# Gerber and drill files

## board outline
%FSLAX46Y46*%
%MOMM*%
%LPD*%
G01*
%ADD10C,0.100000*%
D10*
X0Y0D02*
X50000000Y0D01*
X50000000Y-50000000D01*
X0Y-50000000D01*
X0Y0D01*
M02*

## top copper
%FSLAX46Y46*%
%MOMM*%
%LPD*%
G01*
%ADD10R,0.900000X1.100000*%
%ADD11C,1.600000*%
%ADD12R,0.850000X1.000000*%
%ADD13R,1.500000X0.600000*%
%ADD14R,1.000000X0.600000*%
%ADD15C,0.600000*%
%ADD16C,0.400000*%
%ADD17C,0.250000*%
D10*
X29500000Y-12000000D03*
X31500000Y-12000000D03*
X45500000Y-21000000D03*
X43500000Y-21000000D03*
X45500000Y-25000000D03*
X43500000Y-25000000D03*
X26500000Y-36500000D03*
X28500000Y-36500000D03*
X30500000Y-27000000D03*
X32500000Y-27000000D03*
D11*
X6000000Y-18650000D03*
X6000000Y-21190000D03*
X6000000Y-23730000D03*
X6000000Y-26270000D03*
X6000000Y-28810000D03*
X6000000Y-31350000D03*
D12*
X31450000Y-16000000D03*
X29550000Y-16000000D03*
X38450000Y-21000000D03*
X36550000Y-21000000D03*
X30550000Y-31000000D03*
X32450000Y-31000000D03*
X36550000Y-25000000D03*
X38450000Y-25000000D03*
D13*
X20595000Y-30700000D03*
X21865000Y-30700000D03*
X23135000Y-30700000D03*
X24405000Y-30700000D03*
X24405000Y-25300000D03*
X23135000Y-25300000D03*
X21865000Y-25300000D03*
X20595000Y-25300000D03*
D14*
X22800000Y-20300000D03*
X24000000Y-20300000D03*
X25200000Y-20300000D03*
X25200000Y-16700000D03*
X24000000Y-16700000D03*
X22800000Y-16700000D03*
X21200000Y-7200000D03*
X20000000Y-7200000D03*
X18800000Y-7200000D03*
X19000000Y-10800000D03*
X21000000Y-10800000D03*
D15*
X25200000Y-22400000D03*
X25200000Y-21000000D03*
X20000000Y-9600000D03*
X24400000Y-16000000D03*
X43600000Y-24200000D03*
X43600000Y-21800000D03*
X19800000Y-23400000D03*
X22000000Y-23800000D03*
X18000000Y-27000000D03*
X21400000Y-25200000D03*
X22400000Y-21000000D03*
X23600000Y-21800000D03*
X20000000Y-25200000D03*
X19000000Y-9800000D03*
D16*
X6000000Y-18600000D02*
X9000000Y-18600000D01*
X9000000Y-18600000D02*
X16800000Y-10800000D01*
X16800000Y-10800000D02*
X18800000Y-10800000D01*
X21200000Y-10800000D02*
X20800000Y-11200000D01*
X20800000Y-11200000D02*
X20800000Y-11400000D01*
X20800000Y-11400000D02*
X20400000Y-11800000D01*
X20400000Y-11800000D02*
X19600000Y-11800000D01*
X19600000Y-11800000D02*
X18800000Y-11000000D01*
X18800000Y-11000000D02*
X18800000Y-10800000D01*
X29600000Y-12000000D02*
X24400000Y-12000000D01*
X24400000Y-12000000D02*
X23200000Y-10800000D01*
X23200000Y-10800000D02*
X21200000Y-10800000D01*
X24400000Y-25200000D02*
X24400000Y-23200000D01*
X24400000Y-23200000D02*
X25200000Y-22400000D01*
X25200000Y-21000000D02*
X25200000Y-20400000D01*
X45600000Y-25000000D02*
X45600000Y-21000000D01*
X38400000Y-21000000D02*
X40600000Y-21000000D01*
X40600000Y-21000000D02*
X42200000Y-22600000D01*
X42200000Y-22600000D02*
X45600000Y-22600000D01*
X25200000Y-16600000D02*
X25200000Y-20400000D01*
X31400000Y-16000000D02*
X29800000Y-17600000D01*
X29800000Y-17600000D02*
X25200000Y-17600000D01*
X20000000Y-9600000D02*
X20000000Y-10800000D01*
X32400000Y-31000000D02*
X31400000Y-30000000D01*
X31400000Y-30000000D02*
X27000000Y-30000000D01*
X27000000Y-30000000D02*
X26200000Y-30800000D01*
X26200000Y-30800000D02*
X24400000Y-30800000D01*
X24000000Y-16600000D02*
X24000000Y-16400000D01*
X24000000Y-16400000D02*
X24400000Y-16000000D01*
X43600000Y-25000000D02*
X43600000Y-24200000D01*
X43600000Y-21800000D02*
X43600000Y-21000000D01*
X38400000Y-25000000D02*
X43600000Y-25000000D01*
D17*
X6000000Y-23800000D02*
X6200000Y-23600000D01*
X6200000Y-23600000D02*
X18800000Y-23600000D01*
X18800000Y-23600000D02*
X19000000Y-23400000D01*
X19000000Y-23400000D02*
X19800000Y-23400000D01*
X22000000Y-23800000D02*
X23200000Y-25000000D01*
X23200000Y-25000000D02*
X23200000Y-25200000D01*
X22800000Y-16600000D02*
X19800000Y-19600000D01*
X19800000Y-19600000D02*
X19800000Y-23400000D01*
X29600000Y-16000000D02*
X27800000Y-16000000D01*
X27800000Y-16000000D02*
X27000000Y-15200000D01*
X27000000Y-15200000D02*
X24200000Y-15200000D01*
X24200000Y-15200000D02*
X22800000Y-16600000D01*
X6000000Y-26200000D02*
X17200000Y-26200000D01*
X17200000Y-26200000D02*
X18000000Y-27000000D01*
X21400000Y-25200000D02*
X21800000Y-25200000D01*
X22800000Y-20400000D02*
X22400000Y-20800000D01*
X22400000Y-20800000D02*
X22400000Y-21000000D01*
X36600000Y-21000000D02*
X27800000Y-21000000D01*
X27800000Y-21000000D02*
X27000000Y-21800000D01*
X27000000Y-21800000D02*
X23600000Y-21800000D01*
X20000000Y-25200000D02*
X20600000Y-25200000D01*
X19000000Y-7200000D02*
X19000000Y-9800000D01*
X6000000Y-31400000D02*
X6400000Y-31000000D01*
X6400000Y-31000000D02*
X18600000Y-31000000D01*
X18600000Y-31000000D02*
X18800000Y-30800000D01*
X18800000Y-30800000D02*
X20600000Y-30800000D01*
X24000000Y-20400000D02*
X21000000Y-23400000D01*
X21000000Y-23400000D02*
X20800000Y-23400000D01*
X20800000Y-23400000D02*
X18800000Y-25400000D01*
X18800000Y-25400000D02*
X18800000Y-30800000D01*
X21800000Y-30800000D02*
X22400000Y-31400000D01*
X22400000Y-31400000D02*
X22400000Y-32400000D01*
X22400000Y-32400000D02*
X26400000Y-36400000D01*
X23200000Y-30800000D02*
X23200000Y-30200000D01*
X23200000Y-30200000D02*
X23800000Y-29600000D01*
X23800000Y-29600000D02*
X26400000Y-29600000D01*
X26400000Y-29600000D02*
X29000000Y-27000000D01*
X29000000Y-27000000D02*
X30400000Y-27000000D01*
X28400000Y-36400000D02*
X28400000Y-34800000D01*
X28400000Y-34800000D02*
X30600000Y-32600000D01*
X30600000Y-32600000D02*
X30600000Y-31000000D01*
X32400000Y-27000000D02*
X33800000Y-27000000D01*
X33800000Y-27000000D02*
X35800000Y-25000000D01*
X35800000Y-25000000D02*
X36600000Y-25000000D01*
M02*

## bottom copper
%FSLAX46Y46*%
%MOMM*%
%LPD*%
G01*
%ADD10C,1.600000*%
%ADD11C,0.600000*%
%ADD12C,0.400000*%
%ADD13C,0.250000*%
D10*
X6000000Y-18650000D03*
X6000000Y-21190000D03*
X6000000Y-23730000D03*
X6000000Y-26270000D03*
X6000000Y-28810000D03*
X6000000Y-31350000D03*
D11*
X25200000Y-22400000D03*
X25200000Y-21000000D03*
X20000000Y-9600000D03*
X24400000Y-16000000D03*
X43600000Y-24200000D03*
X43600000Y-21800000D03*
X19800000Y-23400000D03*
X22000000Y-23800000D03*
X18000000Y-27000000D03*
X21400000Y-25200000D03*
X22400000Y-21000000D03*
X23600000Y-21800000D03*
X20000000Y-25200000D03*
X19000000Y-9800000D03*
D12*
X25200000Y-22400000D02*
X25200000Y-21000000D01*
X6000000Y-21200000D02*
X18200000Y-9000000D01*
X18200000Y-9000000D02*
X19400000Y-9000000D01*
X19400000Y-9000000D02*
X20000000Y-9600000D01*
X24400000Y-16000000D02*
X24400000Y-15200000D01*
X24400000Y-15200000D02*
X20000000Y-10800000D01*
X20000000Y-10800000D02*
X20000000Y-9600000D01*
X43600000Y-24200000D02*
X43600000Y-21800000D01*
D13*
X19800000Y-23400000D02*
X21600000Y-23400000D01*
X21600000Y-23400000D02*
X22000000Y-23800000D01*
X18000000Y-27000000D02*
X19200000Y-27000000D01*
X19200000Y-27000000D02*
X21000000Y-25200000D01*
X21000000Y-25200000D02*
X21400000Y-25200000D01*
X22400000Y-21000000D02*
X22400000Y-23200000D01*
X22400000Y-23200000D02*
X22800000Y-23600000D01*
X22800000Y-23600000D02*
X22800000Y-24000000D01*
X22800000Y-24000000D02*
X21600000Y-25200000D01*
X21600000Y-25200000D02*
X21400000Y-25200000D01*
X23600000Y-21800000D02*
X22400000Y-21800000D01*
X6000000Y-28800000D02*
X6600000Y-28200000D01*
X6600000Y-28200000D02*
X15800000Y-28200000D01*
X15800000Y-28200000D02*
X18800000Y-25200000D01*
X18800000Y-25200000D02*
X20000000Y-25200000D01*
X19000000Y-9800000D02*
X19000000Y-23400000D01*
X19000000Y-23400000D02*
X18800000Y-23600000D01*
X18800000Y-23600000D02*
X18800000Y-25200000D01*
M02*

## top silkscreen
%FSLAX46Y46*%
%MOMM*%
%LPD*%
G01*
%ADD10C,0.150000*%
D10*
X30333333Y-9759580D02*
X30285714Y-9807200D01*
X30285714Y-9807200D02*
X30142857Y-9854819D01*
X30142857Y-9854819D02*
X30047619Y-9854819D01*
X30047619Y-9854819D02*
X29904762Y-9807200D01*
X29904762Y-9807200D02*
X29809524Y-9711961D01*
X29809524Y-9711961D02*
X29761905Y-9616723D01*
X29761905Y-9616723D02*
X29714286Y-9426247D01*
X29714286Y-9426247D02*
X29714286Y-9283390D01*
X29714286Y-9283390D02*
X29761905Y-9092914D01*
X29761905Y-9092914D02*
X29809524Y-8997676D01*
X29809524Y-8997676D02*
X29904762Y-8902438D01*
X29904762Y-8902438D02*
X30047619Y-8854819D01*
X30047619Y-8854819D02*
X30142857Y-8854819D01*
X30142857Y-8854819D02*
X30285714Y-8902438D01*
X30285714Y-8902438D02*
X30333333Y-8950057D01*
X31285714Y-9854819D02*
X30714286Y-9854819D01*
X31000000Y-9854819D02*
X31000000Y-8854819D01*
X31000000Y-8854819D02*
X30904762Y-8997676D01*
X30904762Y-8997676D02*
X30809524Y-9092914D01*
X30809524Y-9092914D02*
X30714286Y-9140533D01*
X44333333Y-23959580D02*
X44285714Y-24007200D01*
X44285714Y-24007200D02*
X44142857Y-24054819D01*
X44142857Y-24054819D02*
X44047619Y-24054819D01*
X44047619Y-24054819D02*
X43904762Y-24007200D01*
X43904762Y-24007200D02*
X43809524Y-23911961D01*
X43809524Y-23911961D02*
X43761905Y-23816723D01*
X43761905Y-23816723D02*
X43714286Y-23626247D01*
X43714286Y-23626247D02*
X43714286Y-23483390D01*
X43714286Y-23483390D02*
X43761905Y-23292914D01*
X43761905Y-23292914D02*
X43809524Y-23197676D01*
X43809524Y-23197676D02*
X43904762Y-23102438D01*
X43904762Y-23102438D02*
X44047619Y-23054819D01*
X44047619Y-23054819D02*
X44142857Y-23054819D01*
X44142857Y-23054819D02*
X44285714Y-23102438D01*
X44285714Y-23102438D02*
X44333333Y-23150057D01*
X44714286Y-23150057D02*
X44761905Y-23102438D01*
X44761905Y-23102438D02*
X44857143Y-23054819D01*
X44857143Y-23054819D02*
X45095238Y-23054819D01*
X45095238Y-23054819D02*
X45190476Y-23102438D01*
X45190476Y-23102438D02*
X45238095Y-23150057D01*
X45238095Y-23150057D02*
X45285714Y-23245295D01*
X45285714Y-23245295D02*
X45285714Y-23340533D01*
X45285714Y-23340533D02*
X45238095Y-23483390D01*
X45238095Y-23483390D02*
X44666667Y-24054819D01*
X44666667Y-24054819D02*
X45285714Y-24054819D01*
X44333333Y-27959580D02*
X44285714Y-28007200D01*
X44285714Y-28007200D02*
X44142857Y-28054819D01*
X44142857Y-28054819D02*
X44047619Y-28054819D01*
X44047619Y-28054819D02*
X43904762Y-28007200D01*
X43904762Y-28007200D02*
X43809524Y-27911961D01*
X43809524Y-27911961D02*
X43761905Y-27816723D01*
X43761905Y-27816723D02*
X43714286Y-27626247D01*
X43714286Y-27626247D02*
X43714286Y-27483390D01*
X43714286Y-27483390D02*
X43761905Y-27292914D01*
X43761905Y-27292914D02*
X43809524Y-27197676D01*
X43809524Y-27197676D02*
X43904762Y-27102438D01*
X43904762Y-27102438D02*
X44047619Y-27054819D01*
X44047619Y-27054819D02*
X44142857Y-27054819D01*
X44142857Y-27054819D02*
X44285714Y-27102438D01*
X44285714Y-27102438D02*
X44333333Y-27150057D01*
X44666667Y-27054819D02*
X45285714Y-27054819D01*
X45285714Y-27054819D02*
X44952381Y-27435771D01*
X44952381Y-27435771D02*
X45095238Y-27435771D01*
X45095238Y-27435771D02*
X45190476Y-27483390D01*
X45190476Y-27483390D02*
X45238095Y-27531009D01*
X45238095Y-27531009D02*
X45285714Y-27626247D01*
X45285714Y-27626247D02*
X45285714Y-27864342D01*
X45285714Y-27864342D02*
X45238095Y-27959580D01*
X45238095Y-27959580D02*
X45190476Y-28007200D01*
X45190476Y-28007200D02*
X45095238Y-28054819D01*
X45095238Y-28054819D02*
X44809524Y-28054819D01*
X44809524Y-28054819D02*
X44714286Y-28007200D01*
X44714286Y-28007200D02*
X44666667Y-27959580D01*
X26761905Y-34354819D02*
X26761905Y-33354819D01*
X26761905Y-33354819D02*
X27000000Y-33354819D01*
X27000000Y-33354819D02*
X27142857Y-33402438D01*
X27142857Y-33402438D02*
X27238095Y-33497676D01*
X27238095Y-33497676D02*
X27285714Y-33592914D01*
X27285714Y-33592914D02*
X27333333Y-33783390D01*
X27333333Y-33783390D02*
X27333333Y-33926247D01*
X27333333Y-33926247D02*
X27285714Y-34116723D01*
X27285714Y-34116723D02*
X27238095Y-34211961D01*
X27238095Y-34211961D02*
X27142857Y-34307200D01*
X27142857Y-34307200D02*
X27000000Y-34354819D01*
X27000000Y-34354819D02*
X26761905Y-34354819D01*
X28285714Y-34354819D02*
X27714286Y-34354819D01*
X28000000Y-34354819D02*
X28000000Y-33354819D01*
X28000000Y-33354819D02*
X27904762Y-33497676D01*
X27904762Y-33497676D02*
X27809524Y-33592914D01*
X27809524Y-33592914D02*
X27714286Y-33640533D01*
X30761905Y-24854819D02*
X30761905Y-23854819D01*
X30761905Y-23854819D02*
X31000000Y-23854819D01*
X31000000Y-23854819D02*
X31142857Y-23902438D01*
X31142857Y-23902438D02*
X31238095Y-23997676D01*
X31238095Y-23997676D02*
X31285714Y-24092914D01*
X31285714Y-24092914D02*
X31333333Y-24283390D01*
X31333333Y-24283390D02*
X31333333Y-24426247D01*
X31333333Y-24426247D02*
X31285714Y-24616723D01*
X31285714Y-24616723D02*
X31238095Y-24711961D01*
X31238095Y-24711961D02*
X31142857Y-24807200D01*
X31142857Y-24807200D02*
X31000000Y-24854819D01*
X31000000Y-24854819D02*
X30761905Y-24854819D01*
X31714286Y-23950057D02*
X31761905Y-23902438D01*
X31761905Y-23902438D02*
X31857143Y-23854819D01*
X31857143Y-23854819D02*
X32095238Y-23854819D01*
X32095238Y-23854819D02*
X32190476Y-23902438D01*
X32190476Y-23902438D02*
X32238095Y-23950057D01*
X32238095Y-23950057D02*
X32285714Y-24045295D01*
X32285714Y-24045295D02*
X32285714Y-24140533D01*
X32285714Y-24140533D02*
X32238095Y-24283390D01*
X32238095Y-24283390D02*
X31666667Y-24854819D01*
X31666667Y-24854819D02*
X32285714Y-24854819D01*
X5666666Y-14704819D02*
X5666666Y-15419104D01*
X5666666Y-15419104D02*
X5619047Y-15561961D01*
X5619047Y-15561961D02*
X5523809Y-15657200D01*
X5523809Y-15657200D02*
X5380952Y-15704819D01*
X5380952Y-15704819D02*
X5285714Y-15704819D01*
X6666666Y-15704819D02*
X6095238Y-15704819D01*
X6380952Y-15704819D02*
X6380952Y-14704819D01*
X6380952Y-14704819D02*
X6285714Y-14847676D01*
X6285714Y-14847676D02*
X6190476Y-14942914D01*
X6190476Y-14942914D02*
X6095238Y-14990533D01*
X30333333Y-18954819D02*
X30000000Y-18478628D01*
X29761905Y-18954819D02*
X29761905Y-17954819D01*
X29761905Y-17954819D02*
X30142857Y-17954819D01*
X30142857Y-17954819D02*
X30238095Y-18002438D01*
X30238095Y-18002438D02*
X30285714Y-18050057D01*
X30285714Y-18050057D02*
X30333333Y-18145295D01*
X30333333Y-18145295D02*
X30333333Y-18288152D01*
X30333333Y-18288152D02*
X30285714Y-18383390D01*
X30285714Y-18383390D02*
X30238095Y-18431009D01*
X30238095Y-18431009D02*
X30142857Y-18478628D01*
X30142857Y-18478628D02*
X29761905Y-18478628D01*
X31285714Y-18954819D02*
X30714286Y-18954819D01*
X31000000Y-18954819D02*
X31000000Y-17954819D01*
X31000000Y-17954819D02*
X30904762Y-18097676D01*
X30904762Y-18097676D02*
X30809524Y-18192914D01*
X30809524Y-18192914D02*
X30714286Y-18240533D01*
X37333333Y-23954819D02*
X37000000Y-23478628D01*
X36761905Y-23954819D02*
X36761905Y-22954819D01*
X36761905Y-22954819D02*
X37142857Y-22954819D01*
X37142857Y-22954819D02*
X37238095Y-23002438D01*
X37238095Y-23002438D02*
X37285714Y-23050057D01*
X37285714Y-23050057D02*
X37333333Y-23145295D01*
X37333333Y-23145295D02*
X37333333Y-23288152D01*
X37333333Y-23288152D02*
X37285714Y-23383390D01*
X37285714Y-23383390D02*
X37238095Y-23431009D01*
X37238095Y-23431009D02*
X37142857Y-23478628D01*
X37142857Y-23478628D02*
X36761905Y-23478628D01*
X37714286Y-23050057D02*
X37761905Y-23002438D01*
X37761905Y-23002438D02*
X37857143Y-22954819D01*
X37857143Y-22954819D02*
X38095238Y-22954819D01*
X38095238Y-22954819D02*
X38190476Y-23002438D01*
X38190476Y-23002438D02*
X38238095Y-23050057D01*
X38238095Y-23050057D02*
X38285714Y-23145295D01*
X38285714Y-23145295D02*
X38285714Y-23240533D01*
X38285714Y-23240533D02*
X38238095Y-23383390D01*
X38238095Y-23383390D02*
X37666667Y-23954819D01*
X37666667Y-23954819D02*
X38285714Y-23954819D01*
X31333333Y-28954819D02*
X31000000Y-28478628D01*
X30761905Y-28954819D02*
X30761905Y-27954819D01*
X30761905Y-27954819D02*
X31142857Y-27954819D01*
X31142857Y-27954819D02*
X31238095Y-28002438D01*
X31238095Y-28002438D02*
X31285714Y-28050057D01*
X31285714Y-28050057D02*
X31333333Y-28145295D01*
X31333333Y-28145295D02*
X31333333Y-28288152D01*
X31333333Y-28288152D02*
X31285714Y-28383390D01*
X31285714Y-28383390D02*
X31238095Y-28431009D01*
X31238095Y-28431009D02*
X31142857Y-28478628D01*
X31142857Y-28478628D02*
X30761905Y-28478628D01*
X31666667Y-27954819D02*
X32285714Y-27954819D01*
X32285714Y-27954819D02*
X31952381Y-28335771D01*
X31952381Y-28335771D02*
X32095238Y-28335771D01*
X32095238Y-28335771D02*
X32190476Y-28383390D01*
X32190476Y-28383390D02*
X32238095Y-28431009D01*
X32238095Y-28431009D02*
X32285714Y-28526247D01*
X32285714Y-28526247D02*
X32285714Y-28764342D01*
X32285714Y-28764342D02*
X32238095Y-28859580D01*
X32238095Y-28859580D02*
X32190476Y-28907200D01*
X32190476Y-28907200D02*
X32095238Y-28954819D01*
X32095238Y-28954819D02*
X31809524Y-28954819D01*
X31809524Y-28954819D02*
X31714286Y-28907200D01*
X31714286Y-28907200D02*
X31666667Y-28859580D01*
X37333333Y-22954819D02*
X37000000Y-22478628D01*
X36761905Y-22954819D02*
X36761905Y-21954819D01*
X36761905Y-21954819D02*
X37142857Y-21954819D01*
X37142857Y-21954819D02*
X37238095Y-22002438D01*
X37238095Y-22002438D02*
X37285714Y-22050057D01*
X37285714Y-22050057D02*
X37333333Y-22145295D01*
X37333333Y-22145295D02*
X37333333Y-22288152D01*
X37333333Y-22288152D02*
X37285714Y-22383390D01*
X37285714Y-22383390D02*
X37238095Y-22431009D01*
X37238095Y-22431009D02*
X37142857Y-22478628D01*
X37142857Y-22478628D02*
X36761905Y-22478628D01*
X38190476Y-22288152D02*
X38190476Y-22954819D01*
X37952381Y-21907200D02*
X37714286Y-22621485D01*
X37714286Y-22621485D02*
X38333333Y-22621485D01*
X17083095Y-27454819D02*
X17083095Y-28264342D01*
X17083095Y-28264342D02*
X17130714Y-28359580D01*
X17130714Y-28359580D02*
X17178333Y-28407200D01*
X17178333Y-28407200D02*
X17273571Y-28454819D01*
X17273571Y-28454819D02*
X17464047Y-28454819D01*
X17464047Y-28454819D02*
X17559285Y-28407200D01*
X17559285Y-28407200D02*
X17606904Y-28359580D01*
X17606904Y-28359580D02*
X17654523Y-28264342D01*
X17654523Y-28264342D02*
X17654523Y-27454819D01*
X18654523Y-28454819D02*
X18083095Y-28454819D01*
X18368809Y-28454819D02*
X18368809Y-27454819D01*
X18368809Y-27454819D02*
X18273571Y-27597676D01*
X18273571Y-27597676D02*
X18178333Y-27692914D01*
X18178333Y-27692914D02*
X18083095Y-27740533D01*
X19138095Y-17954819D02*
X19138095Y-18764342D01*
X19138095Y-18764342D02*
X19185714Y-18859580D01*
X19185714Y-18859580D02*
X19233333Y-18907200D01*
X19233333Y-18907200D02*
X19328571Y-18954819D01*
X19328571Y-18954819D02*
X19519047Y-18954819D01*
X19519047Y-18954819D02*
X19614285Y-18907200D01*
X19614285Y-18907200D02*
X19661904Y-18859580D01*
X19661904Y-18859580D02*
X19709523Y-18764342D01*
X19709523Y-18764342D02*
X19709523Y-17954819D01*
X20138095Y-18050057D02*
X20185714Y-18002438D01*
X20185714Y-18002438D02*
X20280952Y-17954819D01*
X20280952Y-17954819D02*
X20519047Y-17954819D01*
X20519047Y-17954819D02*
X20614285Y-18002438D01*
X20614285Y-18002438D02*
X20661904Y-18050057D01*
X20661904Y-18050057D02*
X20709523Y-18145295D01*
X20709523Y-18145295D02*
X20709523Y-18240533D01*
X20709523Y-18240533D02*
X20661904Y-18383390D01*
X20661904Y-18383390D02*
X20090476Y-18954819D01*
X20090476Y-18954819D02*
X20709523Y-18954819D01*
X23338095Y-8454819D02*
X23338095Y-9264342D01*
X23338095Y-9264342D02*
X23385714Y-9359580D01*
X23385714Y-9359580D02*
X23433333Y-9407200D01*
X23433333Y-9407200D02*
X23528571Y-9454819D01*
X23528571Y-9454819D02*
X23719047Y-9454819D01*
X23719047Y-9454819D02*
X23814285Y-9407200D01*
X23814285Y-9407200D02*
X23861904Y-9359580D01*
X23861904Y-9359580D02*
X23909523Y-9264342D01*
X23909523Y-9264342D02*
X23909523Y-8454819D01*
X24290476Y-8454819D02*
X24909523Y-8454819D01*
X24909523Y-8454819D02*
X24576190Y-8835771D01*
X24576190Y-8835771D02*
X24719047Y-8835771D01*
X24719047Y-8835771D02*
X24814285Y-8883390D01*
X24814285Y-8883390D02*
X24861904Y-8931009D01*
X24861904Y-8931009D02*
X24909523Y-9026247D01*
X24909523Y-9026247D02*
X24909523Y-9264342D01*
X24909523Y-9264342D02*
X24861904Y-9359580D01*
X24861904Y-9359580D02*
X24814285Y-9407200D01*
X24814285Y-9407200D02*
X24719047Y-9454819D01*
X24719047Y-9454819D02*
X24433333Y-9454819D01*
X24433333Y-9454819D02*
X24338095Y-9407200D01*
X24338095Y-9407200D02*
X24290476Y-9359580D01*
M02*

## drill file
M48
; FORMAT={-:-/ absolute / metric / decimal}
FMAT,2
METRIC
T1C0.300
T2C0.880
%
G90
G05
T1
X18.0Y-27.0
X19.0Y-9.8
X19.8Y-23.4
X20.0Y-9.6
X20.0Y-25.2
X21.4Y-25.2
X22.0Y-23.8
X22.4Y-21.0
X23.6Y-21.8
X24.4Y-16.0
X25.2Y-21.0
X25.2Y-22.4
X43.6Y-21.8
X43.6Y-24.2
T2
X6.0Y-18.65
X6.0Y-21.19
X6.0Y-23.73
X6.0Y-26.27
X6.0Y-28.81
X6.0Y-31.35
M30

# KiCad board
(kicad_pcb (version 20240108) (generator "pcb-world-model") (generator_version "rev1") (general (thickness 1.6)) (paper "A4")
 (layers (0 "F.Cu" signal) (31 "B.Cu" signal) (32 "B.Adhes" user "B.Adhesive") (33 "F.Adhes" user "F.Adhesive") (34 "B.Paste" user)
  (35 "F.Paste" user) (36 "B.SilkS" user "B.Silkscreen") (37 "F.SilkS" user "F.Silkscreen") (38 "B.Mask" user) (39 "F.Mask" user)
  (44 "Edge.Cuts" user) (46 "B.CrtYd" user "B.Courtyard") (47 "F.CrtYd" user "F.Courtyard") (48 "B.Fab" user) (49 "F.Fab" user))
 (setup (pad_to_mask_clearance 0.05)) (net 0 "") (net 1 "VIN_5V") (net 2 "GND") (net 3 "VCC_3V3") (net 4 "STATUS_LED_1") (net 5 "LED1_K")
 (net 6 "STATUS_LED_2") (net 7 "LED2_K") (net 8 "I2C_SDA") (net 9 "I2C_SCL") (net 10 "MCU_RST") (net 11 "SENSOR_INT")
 (gr_rect (start 0.0 0.0) (end 50.0000 50.0000) (stroke (width 0.1) (type default)) (fill none) (layer "Edge.Cuts"))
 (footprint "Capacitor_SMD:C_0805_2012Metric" (layer "F.Cu") (at 30.5000 12.0000 0)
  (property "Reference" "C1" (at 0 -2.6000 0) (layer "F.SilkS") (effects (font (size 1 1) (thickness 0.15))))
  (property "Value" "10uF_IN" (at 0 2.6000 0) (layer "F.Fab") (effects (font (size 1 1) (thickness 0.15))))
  (pad "1" smd rect (at -1.0000 0.0000) (size 0.9000 1.1000) (layers "F.Cu" "F.Paste" "F.Mask") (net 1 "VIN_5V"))
  (pad "2" smd rect (at 1.0000 0.0000) (size 0.9000 1.1000) (layers "F.Cu" "F.Paste" "F.Mask") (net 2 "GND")))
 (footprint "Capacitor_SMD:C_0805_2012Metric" (layer "F.Cu") (at 44.5000 21.0000 180)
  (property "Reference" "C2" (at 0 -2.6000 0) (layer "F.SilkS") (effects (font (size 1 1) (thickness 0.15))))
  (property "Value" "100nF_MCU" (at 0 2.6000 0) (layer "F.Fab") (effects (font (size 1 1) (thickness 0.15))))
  (pad "1" smd rect (at -1.0000 0.0000) (size 0.9000 1.1000) (layers "F.Cu" "F.Paste" "F.Mask") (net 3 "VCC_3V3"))
  (pad "2" smd rect (at 1.0000 0.0000) (size 0.9000 1.1000) (layers "F.Cu" "F.Paste" "F.Mask") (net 2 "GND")))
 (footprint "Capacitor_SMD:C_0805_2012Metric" (layer "F.Cu") (at 44.5000 25.0000 180)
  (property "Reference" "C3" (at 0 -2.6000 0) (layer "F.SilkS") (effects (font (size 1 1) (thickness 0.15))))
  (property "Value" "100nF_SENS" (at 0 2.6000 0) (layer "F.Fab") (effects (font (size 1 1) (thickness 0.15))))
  (pad "1" smd rect (at -1.0000 0.0000) (size 0.9000 1.1000) (layers "F.Cu" "F.Paste" "F.Mask") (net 3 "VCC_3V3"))
  (pad "2" smd rect (at 1.0000 0.0000) (size 0.9000 1.1000) (layers "F.Cu" "F.Paste" "F.Mask") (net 2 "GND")))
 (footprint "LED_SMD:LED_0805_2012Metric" (layer "F.Cu") (at 27.5000 36.5000 0)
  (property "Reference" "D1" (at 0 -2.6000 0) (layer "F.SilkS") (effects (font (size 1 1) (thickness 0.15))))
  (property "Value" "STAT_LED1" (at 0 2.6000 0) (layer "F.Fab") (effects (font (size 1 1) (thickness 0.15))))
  (pad "1" smd rect (at -1.0000 0.0000) (size 0.9000 1.1000) (layers "F.Cu" "F.Paste" "F.Mask") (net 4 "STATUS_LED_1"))
  (pad "2" smd rect (at 1.0000 0.0000) (size 0.9000 1.1000) (layers "F.Cu" "F.Paste" "F.Mask") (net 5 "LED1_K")))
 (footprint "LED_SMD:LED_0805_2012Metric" (layer "F.Cu") (at 31.5000 27.0000 0)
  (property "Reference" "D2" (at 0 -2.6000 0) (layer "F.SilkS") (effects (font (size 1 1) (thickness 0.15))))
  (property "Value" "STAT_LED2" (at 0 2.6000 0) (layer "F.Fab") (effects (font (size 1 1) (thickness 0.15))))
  (pad "1" smd rect (at -1.0000 0.0000) (size 0.9000 1.1000) (layers "F.Cu" "F.Paste" "F.Mask") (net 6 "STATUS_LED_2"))
  (pad "2" smd rect (at 1.0000 0.0000) (size 0.9000 1.1000) (layers "F.Cu" "F.Paste" "F.Mask") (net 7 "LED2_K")))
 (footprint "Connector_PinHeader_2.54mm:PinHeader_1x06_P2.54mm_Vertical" (layer "F.Cu") (at 6.0000 25.0000 0) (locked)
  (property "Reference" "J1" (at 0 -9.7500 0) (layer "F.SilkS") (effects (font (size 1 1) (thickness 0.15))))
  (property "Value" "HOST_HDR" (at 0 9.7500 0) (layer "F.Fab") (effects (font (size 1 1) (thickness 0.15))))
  (pad "1" thru_hole circle (at 0.0000 -6.3500) (size 1.6000 1.6000) (drill 0.8800) (layers "*.Cu" "*.Mask") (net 1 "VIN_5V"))
  (pad "2" thru_hole circle (at 0.0000 -3.8100) (size 1.6000 1.6000) (drill 0.8800) (layers "*.Cu" "*.Mask") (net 2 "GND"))
  (pad "3" thru_hole circle (at 0.0000 -1.2700) (size 1.6000 1.6000) (drill 0.8800) (layers "*.Cu" "*.Mask") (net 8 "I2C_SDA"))
  (pad "4" thru_hole circle (at 0.0000 1.2700) (size 1.6000 1.6000) (drill 0.8800) (layers "*.Cu" "*.Mask") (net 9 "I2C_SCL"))
  (pad "5" thru_hole circle (at 0.0000 3.8100) (size 1.6000 1.6000) (drill 0.8800) (layers "*.Cu" "*.Mask") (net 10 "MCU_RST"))
  (pad "6" thru_hole circle (at 0.0000 6.3500) (size 1.6000 1.6000) (drill 0.8800) (layers "*.Cu" "*.Mask") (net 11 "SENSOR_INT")))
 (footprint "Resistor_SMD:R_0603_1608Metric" (layer "F.Cu") (at 30.5000 16.0000 180)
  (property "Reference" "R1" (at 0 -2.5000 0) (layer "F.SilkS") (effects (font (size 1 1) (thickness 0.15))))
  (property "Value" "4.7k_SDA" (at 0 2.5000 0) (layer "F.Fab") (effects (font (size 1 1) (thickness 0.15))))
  (pad "1" smd rect (at -0.9500 0.0000) (size 0.8500 1.0000) (layers "F.Cu" "F.Paste" "F.Mask") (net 3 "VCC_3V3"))
  (pad "2" smd rect (at 0.9500 0.0000) (size 0.8500 1.0000) (layers "F.Cu" "F.Paste" "F.Mask") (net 8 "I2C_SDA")))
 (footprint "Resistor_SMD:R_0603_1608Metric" (layer "F.Cu") (at 37.5000 21.0000 180)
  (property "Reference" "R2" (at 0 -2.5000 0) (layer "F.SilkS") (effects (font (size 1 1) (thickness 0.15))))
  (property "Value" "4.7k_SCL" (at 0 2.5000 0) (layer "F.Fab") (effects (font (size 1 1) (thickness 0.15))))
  (pad "1" smd rect (at -0.9500 0.0000) (size 0.8500 1.0000) (layers "F.Cu" "F.Paste" "F.Mask") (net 3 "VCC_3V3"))
  (pad "2" smd rect (at 0.9500 0.0000) (size 0.8500 1.0000) (layers "F.Cu" "F.Paste" "F.Mask") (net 9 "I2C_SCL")))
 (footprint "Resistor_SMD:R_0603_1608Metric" (layer "F.Cu") (at 31.5000 31.0000 0)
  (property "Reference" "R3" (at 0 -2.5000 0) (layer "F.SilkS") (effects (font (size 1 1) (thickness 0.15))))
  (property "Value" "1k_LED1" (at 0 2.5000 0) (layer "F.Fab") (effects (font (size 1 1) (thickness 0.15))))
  (pad "1" smd rect (at -0.9500 0.0000) (size 0.8500 1.0000) (layers "F.Cu" "F.Paste" "F.Mask") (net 5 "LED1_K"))
  (pad "2" smd rect (at 0.9500 0.0000) (size 0.8500 1.0000) (layers "F.Cu" "F.Paste" "F.Mask") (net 2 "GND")))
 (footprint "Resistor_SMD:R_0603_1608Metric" (layer "F.Cu") (at 37.5000 25.0000 0)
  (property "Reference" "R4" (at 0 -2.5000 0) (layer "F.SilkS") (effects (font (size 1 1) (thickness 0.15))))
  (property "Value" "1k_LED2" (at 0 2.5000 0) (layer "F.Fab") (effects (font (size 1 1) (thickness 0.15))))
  (pad "1" smd rect (at -0.9500 0.0000) (size 0.8500 1.0000) (layers "F.Cu" "F.Paste" "F.Mask") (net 7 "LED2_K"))
  (pad "2" smd rect (at 0.9500 0.0000) (size 0.8500 1.0000) (layers "F.Cu" "F.Paste" "F.Mask") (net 2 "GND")))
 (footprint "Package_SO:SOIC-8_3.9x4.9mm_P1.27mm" (layer "F.Cu") (at 22.5000 28.0000 90)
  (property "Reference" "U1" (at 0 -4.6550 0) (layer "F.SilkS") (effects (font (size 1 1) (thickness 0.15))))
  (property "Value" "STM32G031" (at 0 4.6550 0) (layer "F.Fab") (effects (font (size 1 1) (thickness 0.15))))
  (pad "1" smd rect (at -2.7000 -1.9050) (size 1.5000 0.6000) (layers "F.Cu" "F.Paste" "F.Mask") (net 3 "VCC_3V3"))
  (pad "2" smd rect (at -2.7000 -0.6350) (size 1.5000 0.6000) (layers "F.Cu" "F.Paste" "F.Mask") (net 8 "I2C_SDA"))
  (pad "3" smd rect (at -2.7000 0.6350) (size 1.5000 0.6000) (layers "F.Cu" "F.Paste" "F.Mask") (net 9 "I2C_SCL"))
  (pad "4" smd rect (at -2.7000 1.9050) (size 1.5000 0.6000) (layers "F.Cu" "F.Paste" "F.Mask") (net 10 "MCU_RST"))
  (pad "5" smd rect (at 2.7000 1.9050) (size 1.5000 0.6000) (layers "F.Cu" "F.Paste" "F.Mask") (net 11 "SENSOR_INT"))
  (pad "6" smd rect (at 2.7000 0.6350) (size 1.5000 0.6000) (layers "F.Cu" "F.Paste" "F.Mask") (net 4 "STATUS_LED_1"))
  (pad "7" smd rect (at 2.7000 -0.6350) (size 1.5000 0.6000) (layers "F.Cu" "F.Paste" "F.Mask") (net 6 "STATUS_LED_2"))
  (pad "8" smd rect (at 2.7000 -1.9050) (size 1.5000 0.6000) (layers "F.Cu" "F.Paste" "F.Mask") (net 2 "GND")))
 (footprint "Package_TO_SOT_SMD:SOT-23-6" (layer "F.Cu") (at 24.0000 18.5000 90)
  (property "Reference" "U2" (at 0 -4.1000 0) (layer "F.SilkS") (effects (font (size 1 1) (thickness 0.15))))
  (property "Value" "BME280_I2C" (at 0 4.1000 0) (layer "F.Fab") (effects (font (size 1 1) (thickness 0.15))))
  (pad "1" smd rect (at -1.8000 -1.2000) (size 1.0000 0.6000) (layers "F.Cu" "F.Paste" "F.Mask") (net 3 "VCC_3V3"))
  (pad "2" smd rect (at -1.8000 0.0000) (size 1.0000 0.6000) (layers "F.Cu" "F.Paste" "F.Mask") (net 2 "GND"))
  (pad "3" smd rect (at -1.8000 1.2000) (size 1.0000 0.6000) (layers "F.Cu" "F.Paste" "F.Mask") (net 8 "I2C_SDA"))
  (pad "4" smd rect (at 1.8000 1.2000) (size 1.0000 0.6000) (layers "F.Cu" "F.Paste" "F.Mask") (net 9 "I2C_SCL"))
  (pad "5" smd rect (at 1.8000 0.0000) (size 1.0000 0.6000) (layers "F.Cu" "F.Paste" "F.Mask") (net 11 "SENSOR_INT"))
  (pad "6" smd rect (at 1.8000 -1.2000) (size 1.0000 0.6000) (layers "F.Cu" "F.Paste" "F.Mask") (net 3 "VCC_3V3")))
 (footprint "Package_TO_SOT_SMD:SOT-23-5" (layer "F.Cu") (at 20.0000 9.0000 270)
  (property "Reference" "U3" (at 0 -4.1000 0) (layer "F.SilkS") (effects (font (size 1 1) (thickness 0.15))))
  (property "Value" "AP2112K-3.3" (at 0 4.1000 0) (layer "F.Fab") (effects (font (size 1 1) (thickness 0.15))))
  (pad "1" smd rect (at -1.8000 -1.2000) (size 1.0000 0.6000) (layers "F.Cu" "F.Paste" "F.Mask") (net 1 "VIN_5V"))
  (pad "2" smd rect (at -1.8000 0.0000) (size 1.0000 0.6000) (layers "F.Cu" "F.Paste" "F.Mask") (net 2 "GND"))
  (pad "3" smd rect (at -1.8000 1.2000) (size 1.0000 0.6000) (layers "F.Cu" "F.Paste" "F.Mask") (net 1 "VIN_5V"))
  (pad "4" smd rect (at 1.8000 1.0000) (size 1.0000 0.6000) (layers "F.Cu" "F.Paste" "F.Mask") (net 3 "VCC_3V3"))
  (pad "5" smd rect (at 1.8000 -1.0000) (size 1.0000 0.6000) (layers "F.Cu" "F.Paste" "F.Mask") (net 10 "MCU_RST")))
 (segment (start 6.0000 18.6000) (end 9.0000 18.6000) (width 0.4000) (layer "F.Cu") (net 1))
 (segment (start 9.0000 18.6000) (end 16.8000 10.8000) (width 0.4000) (layer "F.Cu") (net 1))
 (segment (start 16.8000 10.8000) (end 18.8000 10.8000) (width 0.4000) (layer "F.Cu") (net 1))
 (segment (start 21.2000 10.8000) (end 20.8000 11.2000) (width 0.4000) (layer "F.Cu") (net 1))
 (segment (start 20.8000 11.2000) (end 20.8000 11.4000) (width 0.4000) (layer "F.Cu") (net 1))
 (segment (start 20.8000 11.4000) (end 20.4000 11.8000) (width 0.4000) (layer "F.Cu") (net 1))
 (segment (start 20.4000 11.8000) (end 19.6000 11.8000) (width 0.4000) (layer "F.Cu") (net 1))
 (segment (start 19.6000 11.8000) (end 18.8000 11.0000) (width 0.4000) (layer "F.Cu") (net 1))
 (segment (start 18.8000 11.0000) (end 18.8000 10.8000) (width 0.4000) (layer "F.Cu") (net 1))
 (segment (start 29.6000 12.0000) (end 24.4000 12.0000) (width 0.4000) (layer "F.Cu") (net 1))
 (segment (start 24.4000 12.0000) (end 23.2000 10.8000) (width 0.4000) (layer "F.Cu") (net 1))
 (segment (start 23.2000 10.8000) (end 21.2000 10.8000) (width 0.4000) (layer "F.Cu") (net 1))
 (segment (start 24.4000 25.2000) (end 24.4000 23.2000) (width 0.4000) (layer "F.Cu") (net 3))
 (segment (start 24.4000 23.2000) (end 25.2000 22.4000) (width 0.4000) (layer "F.Cu") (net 3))
 (segment (start 25.2000 22.4000) (end 25.2000 21.0000) (width 0.4000) (layer "B.Cu") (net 3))
 (segment (start 25.2000 21.0000) (end 25.2000 20.4000) (width 0.4000) (layer "F.Cu") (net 3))
 (segment (start 45.6000 25.0000) (end 45.6000 21.0000) (width 0.4000) (layer "F.Cu") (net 3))
 (segment (start 38.4000 21.0000) (end 40.6000 21.0000) (width 0.4000) (layer "F.Cu") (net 3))
 (segment (start 40.6000 21.0000) (end 42.2000 22.6000) (width 0.4000) (layer "F.Cu") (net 3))
 (segment (start 42.2000 22.6000) (end 45.6000 22.6000) (width 0.4000) (layer "F.Cu") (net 3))
 (segment (start 25.2000 16.6000) (end 25.2000 20.4000) (width 0.4000) (layer "F.Cu") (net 3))
 (segment (start 31.4000 16.0000) (end 29.8000 17.6000) (width 0.4000) (layer "F.Cu") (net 3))
 (segment (start 29.8000 17.6000) (end 25.2000 17.6000) (width 0.4000) (layer "F.Cu") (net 3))
 (segment (start 6.0000 21.2000) (end 18.2000 9.0000) (width 0.4000) (layer "B.Cu") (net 2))
 (segment (start 18.2000 9.0000) (end 19.4000 9.0000) (width 0.4000) (layer "B.Cu") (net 2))
 (segment (start 19.4000 9.0000) (end 20.0000 9.6000) (width 0.4000) (layer "B.Cu") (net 2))
 (segment (start 20.0000 9.6000) (end 20.0000 10.8000) (width 0.4000) (layer "F.Cu") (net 2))
 (segment (start 32.4000 31.0000) (end 31.4000 30.0000) (width 0.4000) (layer "F.Cu") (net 2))
 (segment (start 31.4000 30.0000) (end 27.0000 30.0000) (width 0.4000) (layer "F.Cu") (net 2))
 (segment (start 27.0000 30.0000) (end 26.2000 30.8000) (width 0.4000) (layer "F.Cu") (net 2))
 (segment (start 26.2000 30.8000) (end 24.4000 30.8000) (width 0.4000) (layer "F.Cu") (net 2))
 (segment (start 24.0000 16.6000) (end 24.0000 16.4000) (width 0.4000) (layer "F.Cu") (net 2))
 (segment (start 24.0000 16.4000) (end 24.4000 16.0000) (width 0.4000) (layer "F.Cu") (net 2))
 (segment (start 24.4000 16.0000) (end 24.4000 15.2000) (width 0.4000) (layer "B.Cu") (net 2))
 (segment (start 24.4000 15.2000) (end 20.0000 10.8000) (width 0.4000) (layer "B.Cu") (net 2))
 (segment (start 20.0000 10.8000) (end 20.0000 9.6000) (width 0.4000) (layer "B.Cu") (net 2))
 (segment (start 43.6000 25.0000) (end 43.6000 24.2000) (width 0.4000) (layer "F.Cu") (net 2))
 (segment (start 43.6000 24.2000) (end 43.6000 21.8000) (width 0.4000) (layer "B.Cu") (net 2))
 (segment (start 43.6000 21.8000) (end 43.6000 21.0000) (width 0.4000) (layer "F.Cu") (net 2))
 (segment (start 38.4000 25.0000) (end 43.6000 25.0000) (width 0.4000) (layer "F.Cu") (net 2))
 (segment (start 6.0000 23.8000) (end 6.2000 23.6000) (width 0.2500) (layer "F.Cu") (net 8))
 (segment (start 6.2000 23.6000) (end 18.8000 23.6000) (width 0.2500) (layer "F.Cu") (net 8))
 (segment (start 18.8000 23.6000) (end 19.0000 23.4000) (width 0.2500) (layer "F.Cu") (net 8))
 (segment (start 19.0000 23.4000) (end 19.8000 23.4000) (width 0.2500) (layer "F.Cu") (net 8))
 (segment (start 19.8000 23.4000) (end 21.6000 23.4000) (width 0.2500) (layer "B.Cu") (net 8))
 (segment (start 21.6000 23.4000) (end 22.0000 23.8000) (width 0.2500) (layer "B.Cu") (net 8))
 (segment (start 22.0000 23.8000) (end 23.2000 25.0000) (width 0.2500) (layer "F.Cu") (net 8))
 (segment (start 23.2000 25.0000) (end 23.2000 25.2000) (width 0.2500) (layer "F.Cu") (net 8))
 (segment (start 22.8000 16.6000) (end 19.8000 19.6000) (width 0.2500) (layer "F.Cu") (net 8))
 (segment (start 19.8000 19.6000) (end 19.8000 23.4000) (width 0.2500) (layer "F.Cu") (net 8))
 (segment (start 29.6000 16.0000) (end 27.8000 16.0000) (width 0.2500) (layer "F.Cu") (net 8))
 (segment (start 27.8000 16.0000) (end 27.0000 15.2000) (width 0.2500) (layer "F.Cu") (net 8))
 (segment (start 27.0000 15.2000) (end 24.2000 15.2000) (width 0.2500) (layer "F.Cu") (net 8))
 (segment (start 24.2000 15.2000) (end 22.8000 16.6000) (width 0.2500) (layer "F.Cu") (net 8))
 (segment (start 6.0000 26.2000) (end 17.2000 26.2000) (width 0.2500) (layer "F.Cu") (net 9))
 (segment (start 17.2000 26.2000) (end 18.0000 27.0000) (width 0.2500) (layer "F.Cu") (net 9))
 (segment (start 18.0000 27.0000) (end 19.2000 27.0000) (width 0.2500) (layer "B.Cu") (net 9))
 (segment (start 19.2000 27.0000) (end 21.0000 25.2000) (width 0.2500) (layer "B.Cu") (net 9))
 (segment (start 21.0000 25.2000) (end 21.4000 25.2000) (width 0.2500) (layer "B.Cu") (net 9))
 (segment (start 21.4000 25.2000) (end 21.8000 25.2000) (width 0.2500) (layer "F.Cu") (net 9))
 (segment (start 22.8000 20.4000) (end 22.4000 20.8000) (width 0.2500) (layer "F.Cu") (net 9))
 (segment (start 22.4000 20.8000) (end 22.4000 21.0000) (width 0.2500) (layer "F.Cu") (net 9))
 (segment (start 22.4000 21.0000) (end 22.4000 23.2000) (width 0.2500) (layer "B.Cu") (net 9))
 (segment (start 22.4000 23.2000) (end 22.8000 23.6000) (width 0.2500) (layer "B.Cu") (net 9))
 (segment (start 22.8000 23.6000) (end 22.8000 24.0000) (width 0.2500) (layer "B.Cu") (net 9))
 (segment (start 22.8000 24.0000) (end 21.6000 25.2000) (width 0.2500) (layer "B.Cu") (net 9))
 (segment (start 21.6000 25.2000) (end 21.4000 25.2000) (width 0.2500) (layer "B.Cu") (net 9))
 (segment (start 36.6000 21.0000) (end 27.8000 21.0000) (width 0.2500) (layer "F.Cu") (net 9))
 (segment (start 27.8000 21.0000) (end 27.0000 21.8000) (width 0.2500) (layer "F.Cu") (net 9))
 (segment (start 27.0000 21.8000) (end 23.6000 21.8000) (width 0.2500) (layer "F.Cu") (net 9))
 (segment (start 23.6000 21.8000) (end 22.4000 21.8000) (width 0.2500) (layer "B.Cu") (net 9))
 (segment (start 6.0000 28.8000) (end 6.6000 28.2000) (width 0.2500) (layer "B.Cu") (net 10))
 (segment (start 6.6000 28.2000) (end 15.8000 28.2000) (width 0.2500) (layer "B.Cu") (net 10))
 (segment (start 15.8000 28.2000) (end 18.8000 25.2000) (width 0.2500) (layer "B.Cu") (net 10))
 (segment (start 18.8000 25.2000) (end 20.0000 25.2000) (width 0.2500) (layer "B.Cu") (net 10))
 (segment (start 20.0000 25.2000) (end 20.6000 25.2000) (width 0.2500) (layer "F.Cu") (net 10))
 (segment (start 19.0000 7.2000) (end 19.0000 9.8000) (width 0.2500) (layer "F.Cu") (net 10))
 (segment (start 19.0000 9.8000) (end 19.0000 23.4000) (width 0.2500) (layer "B.Cu") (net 10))
 (segment (start 19.0000 23.4000) (end 18.8000 23.6000) (width 0.2500) (layer "B.Cu") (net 10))
 (segment (start 18.8000 23.6000) (end 18.8000 25.2000) (width 0.2500) (layer "B.Cu") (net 10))
 (segment (start 6.0000 31.4000) (end 6.4000 31.0000) (width 0.2500) (layer "F.Cu") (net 11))
 (segment (start 6.4000 31.0000) (end 18.6000 31.0000) (width 0.2500) (layer "F.Cu") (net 11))
 (segment (start 18.6000 31.0000) (end 18.8000 30.8000) (width 0.2500) (layer "F.Cu") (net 11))
 (segment (start 18.8000 30.8000) (end 20.6000 30.8000) (width 0.2500) (layer "F.Cu") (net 11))
 (segment (start 24.0000 20.4000) (end 21.0000 23.4000) (width 0.2500) (layer "F.Cu") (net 11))
 (segment (start 21.0000 23.4000) (end 20.8000 23.4000) (width 0.2500) (layer "F.Cu") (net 11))
 (segment (start 20.8000 23.4000) (end 18.8000 25.4000) (width 0.2500) (layer "F.Cu") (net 11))
 (segment (start 18.8000 25.4000) (end 18.8000 30.8000) (width 0.2500) (layer "F.Cu") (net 11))
 (segment (start 21.8000 30.8000) (end 22.4000 31.4000) (width 0.2500) (layer "F.Cu") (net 4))
 (segment (start 22.4000 31.4000) (end 22.4000 32.4000) (width 0.2500) (layer "F.Cu") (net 4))
 (segment (start 22.4000 32.4000) (end 26.4000 36.4000) (width 0.2500) (layer "F.Cu") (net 4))
 (segment (start 23.2000 30.8000) (end 23.2000 30.2000) (width 0.2500) (layer "F.Cu") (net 6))
 (segment (start 23.2000 30.2000) (end 23.8000 29.6000) (width 0.2500) (layer "F.Cu") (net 6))
 (segment (start 23.8000 29.6000) (end 26.4000 29.6000) (width 0.2500) (layer "F.Cu") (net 6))
 (segment (start 26.4000 29.6000) (end 29.0000 27.0000) (width 0.2500) (layer "F.Cu") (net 6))
 (segment (start 29.0000 27.0000) (end 30.4000 27.0000) (width 0.2500) (layer "F.Cu") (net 6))
 (segment (start 28.4000 36.4000) (end 28.4000 34.8000) (width 0.2500) (layer "F.Cu") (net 5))
 (segment (start 28.4000 34.8000) (end 30.6000 32.6000) (width 0.2500) (layer "F.Cu") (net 5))
 (segment (start 30.6000 32.6000) (end 30.6000 31.0000) (width 0.2500) (layer "F.Cu") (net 5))
 (segment (start 32.4000 27.0000) (end 33.8000 27.0000) (width 0.2500) (layer "F.Cu") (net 7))
 (segment (start 33.8000 27.0000) (end 35.8000 25.0000) (width 0.2500) (layer "F.Cu") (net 7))
 (segment (start 35.8000 25.0000) (end 36.6000 25.0000) (width 0.2500) (layer "F.Cu") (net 7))
 (via (at 25.2000 22.4000) (size 0.6000) (drill 0.3000) (layers "F.Cu" "B.Cu") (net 3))
 (via (at 25.2000 21.0000) (size 0.6000) (drill 0.3000) (layers "F.Cu" "B.Cu") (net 3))
 (via (at 20.0000 9.6000) (size 0.6000) (drill 0.3000) (layers "F.Cu" "B.Cu") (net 2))
 (via (at 24.4000 16.0000) (size 0.6000) (drill 0.3000) (layers "F.Cu" "B.Cu") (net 2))
 (via (at 43.6000 24.2000) (size 0.6000) (drill 0.3000) (layers "F.Cu" "B.Cu") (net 2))
 (via (at 43.6000 21.8000) (size 0.6000) (drill 0.3000) (layers "F.Cu" "B.Cu") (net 2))
 (via (at 19.8000 23.4000) (size 0.6000) (drill 0.3000) (layers "F.Cu" "B.Cu") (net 8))
 (via (at 22.0000 23.8000) (size 0.6000) (drill 0.3000) (layers "F.Cu" "B.Cu") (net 8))
 (via (at 18.0000 27.0000) (size 0.6000) (drill 0.3000) (layers "F.Cu" "B.Cu") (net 9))
 (via (at 21.4000 25.2000) (size 0.6000) (drill 0.3000) (layers "F.Cu" "B.Cu") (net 9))
 (via (at 22.4000 21.0000) (size 0.6000) (drill 0.3000) (layers "F.Cu" "B.Cu") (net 9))
 (via (at 23.6000 21.8000) (size 0.6000) (drill 0.3000) (layers "F.Cu" "B.Cu") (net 9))
 (via (at 20.0000 25.2000) (size 0.6000) (drill 0.3000) (layers "F.Cu" "B.Cu") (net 10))
 (via (at 19.0000 9.8000) (size 0.6000) (drill 0.3000) (layers "F.Cu" "B.Cu") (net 10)))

